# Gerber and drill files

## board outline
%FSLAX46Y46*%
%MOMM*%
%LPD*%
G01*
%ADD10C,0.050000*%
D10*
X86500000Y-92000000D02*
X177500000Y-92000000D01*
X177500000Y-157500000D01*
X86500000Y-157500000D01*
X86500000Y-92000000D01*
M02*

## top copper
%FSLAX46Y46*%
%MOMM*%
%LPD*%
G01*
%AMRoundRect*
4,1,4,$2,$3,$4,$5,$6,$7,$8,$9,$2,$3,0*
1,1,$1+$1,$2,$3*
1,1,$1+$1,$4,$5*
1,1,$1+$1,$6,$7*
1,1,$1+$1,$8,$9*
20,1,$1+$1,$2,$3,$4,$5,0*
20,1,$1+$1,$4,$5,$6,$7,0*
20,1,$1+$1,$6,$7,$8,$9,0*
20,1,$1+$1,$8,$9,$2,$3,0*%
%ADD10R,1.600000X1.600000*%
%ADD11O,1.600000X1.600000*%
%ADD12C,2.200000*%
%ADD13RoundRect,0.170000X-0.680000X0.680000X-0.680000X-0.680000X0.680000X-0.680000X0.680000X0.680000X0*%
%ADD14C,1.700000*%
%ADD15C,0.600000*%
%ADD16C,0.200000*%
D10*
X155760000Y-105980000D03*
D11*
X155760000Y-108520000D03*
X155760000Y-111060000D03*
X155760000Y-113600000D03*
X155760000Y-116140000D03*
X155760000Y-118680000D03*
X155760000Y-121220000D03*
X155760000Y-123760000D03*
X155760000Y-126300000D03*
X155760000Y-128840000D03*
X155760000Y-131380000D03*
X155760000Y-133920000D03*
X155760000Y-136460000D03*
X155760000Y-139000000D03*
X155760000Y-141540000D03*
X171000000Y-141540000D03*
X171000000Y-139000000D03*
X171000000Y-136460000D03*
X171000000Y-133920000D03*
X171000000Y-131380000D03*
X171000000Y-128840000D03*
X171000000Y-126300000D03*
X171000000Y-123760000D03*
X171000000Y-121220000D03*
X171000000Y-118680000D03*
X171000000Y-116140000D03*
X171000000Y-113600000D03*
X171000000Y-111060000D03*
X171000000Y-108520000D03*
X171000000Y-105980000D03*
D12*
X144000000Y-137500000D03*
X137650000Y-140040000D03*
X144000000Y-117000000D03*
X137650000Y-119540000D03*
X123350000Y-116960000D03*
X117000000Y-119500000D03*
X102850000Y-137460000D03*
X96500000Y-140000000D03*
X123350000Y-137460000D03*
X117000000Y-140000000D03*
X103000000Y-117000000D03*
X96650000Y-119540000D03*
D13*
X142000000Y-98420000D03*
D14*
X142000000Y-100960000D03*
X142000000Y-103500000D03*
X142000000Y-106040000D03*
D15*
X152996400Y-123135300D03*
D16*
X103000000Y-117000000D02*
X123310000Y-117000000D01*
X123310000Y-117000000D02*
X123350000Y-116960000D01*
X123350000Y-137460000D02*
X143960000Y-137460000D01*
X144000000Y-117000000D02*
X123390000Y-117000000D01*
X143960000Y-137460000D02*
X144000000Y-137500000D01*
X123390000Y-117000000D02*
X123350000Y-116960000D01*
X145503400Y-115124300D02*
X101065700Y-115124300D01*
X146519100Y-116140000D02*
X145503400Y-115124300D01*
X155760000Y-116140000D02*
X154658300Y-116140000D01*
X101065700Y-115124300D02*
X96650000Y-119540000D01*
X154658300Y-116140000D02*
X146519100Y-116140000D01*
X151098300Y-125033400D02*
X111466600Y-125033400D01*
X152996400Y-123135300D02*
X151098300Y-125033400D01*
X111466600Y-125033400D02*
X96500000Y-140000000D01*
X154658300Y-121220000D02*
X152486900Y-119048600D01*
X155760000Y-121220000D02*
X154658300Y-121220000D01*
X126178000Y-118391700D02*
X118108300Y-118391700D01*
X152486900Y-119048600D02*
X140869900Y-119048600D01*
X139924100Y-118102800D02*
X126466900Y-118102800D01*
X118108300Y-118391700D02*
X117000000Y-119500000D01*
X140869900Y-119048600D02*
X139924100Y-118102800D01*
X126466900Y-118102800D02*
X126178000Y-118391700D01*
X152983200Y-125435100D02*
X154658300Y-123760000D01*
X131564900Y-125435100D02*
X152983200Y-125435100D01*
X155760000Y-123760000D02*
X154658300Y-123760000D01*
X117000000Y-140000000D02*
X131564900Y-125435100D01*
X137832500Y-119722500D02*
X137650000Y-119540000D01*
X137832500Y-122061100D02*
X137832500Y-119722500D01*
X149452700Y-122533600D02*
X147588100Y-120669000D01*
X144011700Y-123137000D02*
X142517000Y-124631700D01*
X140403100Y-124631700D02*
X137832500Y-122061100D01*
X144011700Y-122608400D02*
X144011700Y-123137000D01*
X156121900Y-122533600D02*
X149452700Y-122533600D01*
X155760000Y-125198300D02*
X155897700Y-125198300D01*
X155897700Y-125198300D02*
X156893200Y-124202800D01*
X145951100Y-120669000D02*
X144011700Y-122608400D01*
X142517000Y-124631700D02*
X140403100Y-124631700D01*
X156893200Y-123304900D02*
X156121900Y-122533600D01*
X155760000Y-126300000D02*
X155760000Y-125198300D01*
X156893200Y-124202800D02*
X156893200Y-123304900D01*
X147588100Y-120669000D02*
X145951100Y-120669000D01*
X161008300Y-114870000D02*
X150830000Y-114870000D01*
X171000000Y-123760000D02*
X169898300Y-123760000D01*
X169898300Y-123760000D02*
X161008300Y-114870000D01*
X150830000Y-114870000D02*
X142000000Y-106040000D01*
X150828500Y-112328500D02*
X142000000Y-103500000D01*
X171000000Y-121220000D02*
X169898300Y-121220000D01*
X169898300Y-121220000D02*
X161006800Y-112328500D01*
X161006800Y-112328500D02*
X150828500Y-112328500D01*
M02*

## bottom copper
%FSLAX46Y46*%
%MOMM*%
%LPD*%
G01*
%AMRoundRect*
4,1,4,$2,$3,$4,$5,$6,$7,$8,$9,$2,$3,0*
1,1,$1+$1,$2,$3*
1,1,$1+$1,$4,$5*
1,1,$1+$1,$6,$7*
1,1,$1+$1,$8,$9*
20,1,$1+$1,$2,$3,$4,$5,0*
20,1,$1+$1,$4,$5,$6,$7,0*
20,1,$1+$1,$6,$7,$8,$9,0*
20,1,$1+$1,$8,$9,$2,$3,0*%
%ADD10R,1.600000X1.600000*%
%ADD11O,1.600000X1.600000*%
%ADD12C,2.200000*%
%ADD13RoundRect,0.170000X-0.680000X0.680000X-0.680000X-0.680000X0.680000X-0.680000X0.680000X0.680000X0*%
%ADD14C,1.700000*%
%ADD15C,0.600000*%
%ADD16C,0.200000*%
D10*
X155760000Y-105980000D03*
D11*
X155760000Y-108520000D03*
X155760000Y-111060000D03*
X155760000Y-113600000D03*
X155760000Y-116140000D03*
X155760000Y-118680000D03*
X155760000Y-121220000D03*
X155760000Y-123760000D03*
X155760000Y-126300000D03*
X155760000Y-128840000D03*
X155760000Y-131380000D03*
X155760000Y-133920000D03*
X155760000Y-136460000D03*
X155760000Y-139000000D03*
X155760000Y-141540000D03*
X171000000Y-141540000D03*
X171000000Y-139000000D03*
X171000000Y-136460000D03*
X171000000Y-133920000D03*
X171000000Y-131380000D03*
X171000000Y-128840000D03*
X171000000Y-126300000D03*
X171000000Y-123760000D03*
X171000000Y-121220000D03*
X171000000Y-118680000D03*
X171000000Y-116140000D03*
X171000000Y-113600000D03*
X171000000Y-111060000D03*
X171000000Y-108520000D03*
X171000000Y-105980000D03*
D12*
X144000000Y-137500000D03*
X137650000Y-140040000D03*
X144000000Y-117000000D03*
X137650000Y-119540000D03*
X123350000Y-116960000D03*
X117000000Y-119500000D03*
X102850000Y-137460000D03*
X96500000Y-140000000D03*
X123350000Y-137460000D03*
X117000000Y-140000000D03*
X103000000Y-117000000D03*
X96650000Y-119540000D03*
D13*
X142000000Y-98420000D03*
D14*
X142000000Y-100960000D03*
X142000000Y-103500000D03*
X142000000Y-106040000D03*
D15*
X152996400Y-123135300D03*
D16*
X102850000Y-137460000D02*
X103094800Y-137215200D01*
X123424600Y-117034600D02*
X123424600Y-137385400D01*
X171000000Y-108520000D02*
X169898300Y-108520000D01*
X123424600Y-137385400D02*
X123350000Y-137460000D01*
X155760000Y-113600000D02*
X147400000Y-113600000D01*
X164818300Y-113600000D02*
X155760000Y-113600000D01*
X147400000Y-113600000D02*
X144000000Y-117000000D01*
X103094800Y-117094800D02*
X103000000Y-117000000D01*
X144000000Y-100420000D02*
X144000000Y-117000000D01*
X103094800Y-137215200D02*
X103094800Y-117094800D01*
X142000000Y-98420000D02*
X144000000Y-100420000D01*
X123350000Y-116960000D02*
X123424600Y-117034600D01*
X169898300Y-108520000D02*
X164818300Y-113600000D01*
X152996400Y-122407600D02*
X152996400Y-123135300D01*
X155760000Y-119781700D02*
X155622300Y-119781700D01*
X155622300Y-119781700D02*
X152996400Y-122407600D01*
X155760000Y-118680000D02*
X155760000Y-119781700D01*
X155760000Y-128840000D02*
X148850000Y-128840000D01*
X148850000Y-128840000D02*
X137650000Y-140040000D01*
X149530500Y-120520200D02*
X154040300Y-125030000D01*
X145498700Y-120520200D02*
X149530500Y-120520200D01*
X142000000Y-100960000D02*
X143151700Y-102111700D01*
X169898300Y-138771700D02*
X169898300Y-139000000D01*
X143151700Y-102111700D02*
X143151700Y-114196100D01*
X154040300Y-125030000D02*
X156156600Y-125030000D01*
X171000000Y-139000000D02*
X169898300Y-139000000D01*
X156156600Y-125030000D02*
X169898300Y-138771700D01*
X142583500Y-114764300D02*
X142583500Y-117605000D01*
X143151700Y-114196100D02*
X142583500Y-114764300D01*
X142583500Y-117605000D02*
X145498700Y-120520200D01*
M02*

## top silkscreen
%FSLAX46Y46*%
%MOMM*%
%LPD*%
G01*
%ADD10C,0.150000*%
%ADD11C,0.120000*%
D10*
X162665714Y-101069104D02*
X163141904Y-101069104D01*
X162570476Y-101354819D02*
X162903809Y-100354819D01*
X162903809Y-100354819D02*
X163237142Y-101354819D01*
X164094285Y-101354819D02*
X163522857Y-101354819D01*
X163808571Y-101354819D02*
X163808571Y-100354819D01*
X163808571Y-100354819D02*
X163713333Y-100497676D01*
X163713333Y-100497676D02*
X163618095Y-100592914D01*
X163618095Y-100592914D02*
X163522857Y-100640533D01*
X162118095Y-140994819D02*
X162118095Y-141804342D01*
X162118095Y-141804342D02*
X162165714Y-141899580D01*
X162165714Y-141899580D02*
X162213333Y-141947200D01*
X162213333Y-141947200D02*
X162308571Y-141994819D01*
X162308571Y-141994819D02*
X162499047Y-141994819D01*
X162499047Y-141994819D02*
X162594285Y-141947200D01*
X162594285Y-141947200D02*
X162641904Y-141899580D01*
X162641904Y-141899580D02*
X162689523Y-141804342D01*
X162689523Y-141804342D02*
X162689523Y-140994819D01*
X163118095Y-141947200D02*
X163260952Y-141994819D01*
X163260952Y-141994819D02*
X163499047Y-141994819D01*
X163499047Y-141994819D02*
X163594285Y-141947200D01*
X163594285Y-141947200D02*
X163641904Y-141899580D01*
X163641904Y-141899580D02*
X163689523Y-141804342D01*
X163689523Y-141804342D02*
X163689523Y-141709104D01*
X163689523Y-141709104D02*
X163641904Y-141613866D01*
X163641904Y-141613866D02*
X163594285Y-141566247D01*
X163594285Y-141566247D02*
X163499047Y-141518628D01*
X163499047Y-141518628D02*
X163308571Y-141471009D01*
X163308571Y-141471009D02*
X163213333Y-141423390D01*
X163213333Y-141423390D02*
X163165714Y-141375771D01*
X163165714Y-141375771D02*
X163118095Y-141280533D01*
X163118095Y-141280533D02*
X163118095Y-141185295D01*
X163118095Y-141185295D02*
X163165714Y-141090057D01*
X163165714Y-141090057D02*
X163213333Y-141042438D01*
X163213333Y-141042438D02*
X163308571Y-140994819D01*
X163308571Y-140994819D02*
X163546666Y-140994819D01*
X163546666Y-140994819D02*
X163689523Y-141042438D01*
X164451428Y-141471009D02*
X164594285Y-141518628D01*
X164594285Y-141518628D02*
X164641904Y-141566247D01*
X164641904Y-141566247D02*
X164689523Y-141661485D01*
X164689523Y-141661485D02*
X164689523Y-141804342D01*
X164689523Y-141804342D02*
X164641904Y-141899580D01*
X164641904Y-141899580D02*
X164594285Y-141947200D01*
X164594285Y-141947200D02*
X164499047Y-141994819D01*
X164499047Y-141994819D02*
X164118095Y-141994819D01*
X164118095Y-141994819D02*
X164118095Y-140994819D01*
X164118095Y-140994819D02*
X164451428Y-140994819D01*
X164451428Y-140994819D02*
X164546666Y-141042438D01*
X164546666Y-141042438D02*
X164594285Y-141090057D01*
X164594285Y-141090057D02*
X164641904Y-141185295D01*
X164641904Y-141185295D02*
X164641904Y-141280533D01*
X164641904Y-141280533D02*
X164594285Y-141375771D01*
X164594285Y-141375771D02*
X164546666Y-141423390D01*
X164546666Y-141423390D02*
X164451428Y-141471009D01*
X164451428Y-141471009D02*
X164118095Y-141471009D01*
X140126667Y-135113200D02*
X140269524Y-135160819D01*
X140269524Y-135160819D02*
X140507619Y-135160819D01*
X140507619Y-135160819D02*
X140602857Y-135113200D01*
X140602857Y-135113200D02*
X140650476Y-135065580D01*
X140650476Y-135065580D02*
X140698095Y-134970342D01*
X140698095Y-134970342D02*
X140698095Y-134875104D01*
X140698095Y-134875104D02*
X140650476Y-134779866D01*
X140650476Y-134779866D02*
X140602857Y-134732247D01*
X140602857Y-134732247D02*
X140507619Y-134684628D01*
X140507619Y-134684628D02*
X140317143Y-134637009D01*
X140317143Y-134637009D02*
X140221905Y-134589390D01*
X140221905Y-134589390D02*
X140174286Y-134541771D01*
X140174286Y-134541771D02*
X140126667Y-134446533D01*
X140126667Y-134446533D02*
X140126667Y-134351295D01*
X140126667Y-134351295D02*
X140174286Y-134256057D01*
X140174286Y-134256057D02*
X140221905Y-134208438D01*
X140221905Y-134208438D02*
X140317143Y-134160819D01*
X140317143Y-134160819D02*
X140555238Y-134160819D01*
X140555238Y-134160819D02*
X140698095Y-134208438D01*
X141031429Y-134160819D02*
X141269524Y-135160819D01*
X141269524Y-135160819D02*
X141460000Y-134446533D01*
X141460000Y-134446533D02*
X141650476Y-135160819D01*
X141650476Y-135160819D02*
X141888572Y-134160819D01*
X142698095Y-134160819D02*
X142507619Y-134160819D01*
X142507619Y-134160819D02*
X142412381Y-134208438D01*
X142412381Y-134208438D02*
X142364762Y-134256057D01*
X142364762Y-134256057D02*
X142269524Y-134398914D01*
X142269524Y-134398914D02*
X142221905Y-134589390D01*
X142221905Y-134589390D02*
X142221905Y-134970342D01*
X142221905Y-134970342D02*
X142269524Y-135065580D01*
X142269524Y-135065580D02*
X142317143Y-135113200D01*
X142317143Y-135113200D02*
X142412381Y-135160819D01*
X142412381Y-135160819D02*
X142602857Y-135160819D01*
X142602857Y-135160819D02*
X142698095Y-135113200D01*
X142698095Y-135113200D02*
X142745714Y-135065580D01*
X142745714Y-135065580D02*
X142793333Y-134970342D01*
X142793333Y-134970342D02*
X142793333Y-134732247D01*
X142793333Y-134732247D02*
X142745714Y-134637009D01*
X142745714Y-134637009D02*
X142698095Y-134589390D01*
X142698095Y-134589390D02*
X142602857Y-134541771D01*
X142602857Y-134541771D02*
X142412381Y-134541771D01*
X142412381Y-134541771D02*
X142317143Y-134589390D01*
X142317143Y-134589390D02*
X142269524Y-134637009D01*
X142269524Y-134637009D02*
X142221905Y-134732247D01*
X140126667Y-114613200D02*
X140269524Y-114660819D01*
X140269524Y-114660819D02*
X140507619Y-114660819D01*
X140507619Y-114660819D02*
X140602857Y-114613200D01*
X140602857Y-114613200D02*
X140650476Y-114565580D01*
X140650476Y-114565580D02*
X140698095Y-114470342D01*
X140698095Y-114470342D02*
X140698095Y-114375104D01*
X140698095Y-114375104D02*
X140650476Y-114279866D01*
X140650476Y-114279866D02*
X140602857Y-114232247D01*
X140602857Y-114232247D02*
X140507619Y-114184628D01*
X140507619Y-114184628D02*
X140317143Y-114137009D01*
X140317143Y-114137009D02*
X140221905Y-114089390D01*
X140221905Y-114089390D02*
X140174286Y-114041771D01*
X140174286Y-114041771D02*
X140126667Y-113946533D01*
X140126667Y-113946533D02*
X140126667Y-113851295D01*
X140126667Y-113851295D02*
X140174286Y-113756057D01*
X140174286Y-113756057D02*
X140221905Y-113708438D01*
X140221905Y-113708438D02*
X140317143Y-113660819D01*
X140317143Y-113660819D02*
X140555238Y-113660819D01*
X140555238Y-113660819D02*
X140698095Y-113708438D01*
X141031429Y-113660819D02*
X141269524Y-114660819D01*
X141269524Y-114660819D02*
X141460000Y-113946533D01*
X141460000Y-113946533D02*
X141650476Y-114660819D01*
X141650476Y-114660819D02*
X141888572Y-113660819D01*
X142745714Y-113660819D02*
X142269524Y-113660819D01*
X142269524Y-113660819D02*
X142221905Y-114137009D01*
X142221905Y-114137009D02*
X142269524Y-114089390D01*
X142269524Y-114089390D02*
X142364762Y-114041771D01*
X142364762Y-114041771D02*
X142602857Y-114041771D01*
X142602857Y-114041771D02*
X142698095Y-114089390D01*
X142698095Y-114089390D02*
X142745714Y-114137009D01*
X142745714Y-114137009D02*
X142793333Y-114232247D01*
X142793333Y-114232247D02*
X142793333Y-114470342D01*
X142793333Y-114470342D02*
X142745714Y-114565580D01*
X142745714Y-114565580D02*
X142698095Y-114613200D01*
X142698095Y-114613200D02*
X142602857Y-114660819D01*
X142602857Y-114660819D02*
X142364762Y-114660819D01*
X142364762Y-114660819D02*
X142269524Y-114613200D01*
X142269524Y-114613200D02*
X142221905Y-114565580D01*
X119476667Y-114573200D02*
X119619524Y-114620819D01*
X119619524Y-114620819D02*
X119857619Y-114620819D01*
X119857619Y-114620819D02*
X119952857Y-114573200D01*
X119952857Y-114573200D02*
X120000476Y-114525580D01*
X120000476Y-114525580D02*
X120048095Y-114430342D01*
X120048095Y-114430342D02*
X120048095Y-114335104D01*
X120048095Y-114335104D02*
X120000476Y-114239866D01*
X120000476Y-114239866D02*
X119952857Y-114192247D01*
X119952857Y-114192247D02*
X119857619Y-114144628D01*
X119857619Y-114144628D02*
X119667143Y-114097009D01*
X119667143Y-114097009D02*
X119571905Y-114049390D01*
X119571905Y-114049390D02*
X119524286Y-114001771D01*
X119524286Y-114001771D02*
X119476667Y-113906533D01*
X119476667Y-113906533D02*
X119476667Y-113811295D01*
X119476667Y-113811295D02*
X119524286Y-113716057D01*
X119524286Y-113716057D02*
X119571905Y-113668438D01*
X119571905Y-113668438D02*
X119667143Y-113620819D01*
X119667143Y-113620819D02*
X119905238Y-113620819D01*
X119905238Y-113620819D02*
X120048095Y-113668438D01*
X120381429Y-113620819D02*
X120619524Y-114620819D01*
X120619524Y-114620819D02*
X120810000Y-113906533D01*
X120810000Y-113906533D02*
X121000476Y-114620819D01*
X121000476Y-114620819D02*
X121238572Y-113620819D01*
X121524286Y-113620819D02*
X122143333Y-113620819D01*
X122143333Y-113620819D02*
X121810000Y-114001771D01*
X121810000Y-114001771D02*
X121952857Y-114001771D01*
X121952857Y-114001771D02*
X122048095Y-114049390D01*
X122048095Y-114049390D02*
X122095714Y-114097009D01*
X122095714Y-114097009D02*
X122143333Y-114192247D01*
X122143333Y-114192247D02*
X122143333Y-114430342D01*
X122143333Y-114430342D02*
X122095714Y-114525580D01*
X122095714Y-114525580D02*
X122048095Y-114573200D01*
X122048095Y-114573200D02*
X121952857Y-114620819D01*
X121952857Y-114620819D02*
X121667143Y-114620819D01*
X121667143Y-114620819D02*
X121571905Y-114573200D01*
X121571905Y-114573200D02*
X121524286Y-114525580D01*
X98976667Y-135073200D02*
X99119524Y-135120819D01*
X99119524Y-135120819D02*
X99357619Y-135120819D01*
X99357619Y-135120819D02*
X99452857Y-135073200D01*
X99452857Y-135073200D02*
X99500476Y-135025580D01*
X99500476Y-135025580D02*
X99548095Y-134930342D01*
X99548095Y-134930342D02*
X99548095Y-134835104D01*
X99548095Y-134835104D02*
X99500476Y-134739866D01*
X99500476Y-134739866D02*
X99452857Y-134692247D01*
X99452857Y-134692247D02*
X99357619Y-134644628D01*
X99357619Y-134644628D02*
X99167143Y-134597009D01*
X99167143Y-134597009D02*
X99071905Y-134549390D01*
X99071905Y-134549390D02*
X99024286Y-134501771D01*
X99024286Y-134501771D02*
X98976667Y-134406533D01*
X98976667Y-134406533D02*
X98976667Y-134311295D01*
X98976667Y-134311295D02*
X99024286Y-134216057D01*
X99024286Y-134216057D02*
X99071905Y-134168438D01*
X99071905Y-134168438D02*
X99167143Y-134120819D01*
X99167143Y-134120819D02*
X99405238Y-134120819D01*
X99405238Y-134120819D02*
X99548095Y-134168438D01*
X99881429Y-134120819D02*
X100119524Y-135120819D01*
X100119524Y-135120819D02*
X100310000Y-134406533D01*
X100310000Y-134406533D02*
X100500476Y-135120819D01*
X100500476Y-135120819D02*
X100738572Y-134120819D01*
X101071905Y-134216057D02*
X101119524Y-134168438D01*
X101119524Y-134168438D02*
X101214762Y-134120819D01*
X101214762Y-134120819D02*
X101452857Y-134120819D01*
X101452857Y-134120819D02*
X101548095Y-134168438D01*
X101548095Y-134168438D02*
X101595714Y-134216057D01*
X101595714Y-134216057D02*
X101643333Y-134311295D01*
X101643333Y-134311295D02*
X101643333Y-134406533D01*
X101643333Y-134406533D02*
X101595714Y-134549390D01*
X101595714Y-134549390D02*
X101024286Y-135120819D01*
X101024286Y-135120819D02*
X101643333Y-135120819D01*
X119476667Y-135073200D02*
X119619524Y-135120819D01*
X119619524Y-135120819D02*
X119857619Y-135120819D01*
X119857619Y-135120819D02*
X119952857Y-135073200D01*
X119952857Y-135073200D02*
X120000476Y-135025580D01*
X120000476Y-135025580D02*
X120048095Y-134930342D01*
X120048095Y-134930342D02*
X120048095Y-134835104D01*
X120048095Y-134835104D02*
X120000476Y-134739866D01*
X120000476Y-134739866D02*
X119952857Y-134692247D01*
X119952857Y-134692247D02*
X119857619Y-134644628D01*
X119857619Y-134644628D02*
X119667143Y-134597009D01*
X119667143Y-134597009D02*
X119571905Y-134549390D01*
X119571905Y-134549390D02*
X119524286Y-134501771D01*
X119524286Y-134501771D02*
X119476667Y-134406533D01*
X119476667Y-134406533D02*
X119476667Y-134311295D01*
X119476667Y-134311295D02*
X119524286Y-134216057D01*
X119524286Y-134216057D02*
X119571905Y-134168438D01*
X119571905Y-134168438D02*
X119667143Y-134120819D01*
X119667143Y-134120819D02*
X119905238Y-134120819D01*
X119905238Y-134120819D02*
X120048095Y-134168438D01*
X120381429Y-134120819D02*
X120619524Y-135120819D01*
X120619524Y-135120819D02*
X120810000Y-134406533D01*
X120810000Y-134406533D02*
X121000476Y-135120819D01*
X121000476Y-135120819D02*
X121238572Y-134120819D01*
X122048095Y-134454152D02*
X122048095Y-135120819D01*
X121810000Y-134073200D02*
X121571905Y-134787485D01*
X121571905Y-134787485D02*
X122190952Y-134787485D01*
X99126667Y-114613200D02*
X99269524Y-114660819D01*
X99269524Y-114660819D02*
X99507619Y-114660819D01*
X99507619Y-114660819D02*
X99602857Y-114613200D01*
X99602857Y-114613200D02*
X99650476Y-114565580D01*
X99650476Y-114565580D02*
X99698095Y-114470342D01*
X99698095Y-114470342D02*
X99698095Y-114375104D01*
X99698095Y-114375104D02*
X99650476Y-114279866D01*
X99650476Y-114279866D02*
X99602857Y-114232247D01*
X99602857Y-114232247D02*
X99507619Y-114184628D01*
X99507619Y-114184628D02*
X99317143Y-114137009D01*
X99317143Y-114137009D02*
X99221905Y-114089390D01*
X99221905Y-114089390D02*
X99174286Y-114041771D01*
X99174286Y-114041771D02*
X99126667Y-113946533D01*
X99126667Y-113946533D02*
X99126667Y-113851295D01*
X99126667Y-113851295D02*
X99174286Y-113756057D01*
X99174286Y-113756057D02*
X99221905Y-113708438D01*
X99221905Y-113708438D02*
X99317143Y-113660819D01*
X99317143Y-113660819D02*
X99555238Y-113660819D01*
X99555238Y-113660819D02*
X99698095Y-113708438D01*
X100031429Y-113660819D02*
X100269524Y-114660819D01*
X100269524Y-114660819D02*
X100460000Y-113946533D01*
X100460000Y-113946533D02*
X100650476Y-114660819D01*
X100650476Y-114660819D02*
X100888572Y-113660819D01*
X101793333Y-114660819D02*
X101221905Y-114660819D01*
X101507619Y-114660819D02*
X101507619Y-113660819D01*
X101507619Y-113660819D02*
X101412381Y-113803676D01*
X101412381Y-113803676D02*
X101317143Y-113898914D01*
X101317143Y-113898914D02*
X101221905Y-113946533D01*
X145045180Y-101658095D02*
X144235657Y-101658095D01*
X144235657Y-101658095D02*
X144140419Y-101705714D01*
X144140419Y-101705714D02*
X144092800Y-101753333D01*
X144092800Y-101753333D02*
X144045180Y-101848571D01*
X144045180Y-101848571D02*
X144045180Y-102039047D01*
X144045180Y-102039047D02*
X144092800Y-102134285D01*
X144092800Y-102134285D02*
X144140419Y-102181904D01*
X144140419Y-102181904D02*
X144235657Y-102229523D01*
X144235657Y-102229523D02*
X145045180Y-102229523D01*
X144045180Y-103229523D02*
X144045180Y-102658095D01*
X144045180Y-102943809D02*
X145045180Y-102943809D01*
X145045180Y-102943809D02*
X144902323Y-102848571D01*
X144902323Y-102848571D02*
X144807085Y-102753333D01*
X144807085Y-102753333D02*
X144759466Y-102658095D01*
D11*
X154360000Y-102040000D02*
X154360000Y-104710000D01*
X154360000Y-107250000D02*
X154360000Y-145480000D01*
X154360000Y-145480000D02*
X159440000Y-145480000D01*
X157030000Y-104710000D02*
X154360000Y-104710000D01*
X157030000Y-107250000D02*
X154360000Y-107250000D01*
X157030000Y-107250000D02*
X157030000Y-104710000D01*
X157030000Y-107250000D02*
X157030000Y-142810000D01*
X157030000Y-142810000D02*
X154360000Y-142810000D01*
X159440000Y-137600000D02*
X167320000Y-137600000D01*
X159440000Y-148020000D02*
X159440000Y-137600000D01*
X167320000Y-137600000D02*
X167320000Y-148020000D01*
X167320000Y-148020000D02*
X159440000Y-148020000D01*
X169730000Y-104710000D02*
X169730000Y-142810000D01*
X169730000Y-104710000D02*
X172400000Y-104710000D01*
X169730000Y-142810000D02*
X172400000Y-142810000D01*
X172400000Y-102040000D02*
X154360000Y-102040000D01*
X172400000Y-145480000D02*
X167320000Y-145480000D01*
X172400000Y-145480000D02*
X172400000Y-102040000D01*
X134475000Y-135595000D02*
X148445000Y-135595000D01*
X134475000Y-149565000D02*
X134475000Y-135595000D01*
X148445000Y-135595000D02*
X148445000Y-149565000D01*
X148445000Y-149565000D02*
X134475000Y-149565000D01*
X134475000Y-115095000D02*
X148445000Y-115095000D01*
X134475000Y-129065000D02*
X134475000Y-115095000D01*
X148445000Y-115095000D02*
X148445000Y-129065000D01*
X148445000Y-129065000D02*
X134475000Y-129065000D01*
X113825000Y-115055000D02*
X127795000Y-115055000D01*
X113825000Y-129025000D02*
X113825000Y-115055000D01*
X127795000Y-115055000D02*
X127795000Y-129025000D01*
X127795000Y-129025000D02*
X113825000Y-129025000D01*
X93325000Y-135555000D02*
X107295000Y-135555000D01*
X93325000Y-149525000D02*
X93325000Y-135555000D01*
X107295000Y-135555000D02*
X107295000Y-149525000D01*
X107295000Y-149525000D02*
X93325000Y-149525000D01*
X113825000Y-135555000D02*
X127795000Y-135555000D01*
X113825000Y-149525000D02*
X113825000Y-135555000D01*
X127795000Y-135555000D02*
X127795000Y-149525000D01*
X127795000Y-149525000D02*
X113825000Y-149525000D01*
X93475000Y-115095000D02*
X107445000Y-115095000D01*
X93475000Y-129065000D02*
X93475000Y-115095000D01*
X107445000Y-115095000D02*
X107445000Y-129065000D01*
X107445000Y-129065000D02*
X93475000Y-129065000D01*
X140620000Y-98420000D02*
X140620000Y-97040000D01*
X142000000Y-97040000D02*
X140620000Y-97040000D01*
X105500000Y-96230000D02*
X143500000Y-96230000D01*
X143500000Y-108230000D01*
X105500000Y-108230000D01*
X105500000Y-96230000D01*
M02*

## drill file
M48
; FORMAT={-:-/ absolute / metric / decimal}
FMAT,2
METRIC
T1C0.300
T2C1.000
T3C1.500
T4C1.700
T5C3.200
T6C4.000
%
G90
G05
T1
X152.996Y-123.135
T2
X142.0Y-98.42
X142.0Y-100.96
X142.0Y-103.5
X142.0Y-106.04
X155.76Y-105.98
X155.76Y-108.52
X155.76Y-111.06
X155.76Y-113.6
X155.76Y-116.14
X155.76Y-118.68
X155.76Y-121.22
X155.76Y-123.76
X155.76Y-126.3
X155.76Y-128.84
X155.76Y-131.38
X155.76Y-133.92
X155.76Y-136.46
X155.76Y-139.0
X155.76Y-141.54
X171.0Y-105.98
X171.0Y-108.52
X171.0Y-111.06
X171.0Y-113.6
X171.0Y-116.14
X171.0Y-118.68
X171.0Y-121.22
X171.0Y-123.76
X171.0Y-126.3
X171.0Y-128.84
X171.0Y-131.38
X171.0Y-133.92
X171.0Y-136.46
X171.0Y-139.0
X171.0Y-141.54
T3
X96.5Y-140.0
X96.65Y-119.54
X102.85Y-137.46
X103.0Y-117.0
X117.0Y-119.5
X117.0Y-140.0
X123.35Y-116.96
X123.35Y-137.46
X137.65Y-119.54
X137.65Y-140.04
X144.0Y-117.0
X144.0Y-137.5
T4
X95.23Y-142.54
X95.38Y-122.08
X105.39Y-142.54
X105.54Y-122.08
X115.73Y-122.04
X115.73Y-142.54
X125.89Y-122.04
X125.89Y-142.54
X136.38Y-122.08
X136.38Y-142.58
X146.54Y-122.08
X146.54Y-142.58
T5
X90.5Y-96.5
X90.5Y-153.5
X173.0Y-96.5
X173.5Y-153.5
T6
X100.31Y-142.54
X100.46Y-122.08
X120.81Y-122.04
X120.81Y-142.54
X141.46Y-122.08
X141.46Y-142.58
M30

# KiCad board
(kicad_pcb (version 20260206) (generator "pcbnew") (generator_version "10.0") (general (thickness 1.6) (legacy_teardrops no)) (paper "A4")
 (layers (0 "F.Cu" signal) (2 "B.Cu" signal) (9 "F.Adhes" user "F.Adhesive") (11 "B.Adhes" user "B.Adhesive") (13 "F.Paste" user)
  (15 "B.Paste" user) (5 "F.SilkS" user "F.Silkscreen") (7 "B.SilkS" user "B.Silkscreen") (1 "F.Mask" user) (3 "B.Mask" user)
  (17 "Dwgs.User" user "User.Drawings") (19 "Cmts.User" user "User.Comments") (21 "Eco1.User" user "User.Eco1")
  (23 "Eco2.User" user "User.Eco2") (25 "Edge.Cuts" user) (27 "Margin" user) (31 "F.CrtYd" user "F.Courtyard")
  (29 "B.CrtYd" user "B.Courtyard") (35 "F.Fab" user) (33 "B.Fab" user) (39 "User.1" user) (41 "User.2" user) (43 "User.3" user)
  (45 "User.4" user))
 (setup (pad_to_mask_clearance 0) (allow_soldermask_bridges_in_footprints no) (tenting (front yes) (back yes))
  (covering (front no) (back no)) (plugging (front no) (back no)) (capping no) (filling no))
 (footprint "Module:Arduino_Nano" (layer "F.Cu") (at 155.76 105.98)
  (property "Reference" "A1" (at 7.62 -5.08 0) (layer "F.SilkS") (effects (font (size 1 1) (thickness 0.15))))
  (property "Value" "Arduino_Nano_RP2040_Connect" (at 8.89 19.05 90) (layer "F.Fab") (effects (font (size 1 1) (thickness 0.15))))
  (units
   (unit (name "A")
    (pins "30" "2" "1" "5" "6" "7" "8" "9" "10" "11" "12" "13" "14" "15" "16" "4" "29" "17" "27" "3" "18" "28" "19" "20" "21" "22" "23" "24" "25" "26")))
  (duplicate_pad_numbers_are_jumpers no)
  (fp_line (start -1.4 -3.94) (end -1.4 -1.27) (stroke (width 0.12) (type solid)) (layer "F.SilkS"))
  (fp_line (start -1.4 1.27) (end -1.4 39.5) (stroke (width 0.12) (type solid)) (layer "F.SilkS"))
  (fp_line (start -1.4 39.5) (end 3.68 39.5) (stroke (width 0.12) (type solid)) (layer "F.SilkS"))
  (fp_line (start 1.27 -1.27) (end -1.4 -1.27) (stroke (width 0.12) (type solid)) (layer "F.SilkS"))
  (fp_line (start 1.27 1.27) (end -1.4 1.27) (stroke (width 0.12) (type solid)) (layer "F.SilkS"))
  (fp_line (start 1.27 1.27) (end 1.27 -1.27) (stroke (width 0.12) (type solid)) (layer "F.SilkS"))
  (fp_line (start 1.27 1.27) (end 1.27 36.83) (stroke (width 0.12) (type solid)) (layer "F.SilkS"))
  (fp_line (start 1.27 36.83) (end -1.4 36.83) (stroke (width 0.12) (type solid)) (layer "F.SilkS"))
  (fp_line (start 3.68 31.62) (end 11.56 31.62) (stroke (width 0.12) (type solid)) (layer "F.SilkS"))
  (fp_line (start 3.68 42.04) (end 3.68 31.62) (stroke (width 0.12) (type solid)) (layer "F.SilkS"))
  (fp_line (start 11.56 31.62) (end 11.56 42.04) (stroke (width 0.12) (type solid)) (layer "F.SilkS"))
  (fp_line (start 11.56 42.04) (end 3.68 42.04) (stroke (width 0.12) (type solid)) (layer "F.SilkS"))
  (fp_line (start 13.97 -1.27) (end 13.97 36.83) (stroke (width 0.12) (type solid)) (layer "F.SilkS"))
  (fp_line (start 13.97 -1.27) (end 16.64 -1.27) (stroke (width 0.12) (type solid)) (layer "F.SilkS"))
  (fp_line (start 13.97 36.83) (end 16.64 36.83) (stroke (width 0.12) (type solid)) (layer "F.SilkS"))
  (fp_line (start 16.64 -3.94) (end -1.4 -3.94) (stroke (width 0.12) (type solid)) (layer "F.SilkS"))
  (fp_line (start 16.64 39.5) (end 11.56 39.5) (stroke (width 0.12) (type solid)) (layer "F.SilkS"))
  (fp_line (start 16.64 39.5) (end 16.64 -3.94) (stroke (width 0.12) (type solid)) (layer "F.SilkS"))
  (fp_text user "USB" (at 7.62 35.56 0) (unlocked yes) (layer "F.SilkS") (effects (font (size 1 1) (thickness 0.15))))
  (pad "1" thru_hole rect (at 0 0) (size 1.6 1.6) (drill 1) (layers "*.Cu" "*.Mask") (remove_unused_layers no)
   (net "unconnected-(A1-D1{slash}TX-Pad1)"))
  (pad "2" thru_hole oval (at 0 2.54) (size 1.6 1.6) (drill 1) (layers "*.Cu" "*.Mask") (remove_unused_layers no)
   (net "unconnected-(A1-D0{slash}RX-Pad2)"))
  (pad "3" thru_hole oval (at 0 5.08) (size 1.6 1.6) (drill 1) (layers "*.Cu" "*.Mask") (remove_unused_layers no)
   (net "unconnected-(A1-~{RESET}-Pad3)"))
  (pad "4" thru_hole oval (at 0 7.62) (size 1.6 1.6) (drill 1) (layers "*.Cu" "*.Mask") (remove_unused_layers no) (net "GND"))
  (pad "5" thru_hole oval (at 0 10.16) (size 1.6 1.6) (drill 1) (layers "*.Cu" "*.Mask") (remove_unused_layers no) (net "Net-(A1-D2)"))
  (pad "6" thru_hole oval (at 0 12.7) (size 1.6 1.6) (drill 1) (layers "*.Cu" "*.Mask") (remove_unused_layers no) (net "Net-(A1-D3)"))
  (pad "7" thru_hole oval (at 0 15.24) (size 1.6 1.6) (drill 1) (layers "*.Cu" "*.Mask") (remove_unused_layers no) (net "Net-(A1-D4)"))
  (pad "8" thru_hole oval (at 0 17.78) (size 1.6 1.6) (drill 1) (layers "*.Cu" "*.Mask") (remove_unused_layers no) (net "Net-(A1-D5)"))
  (pad "9" thru_hole oval (at 0 20.32) (size 1.6 1.6) (drill 1) (layers "*.Cu" "*.Mask") (remove_unused_layers no) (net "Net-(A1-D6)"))
  (pad "10" thru_hole oval (at 0 22.86) (size 1.6 1.6) (drill 1) (layers "*.Cu" "*.Mask") (remove_unused_layers no) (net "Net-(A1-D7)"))
  (pad "11" thru_hole oval (at 0 25.4) (size 1.6 1.6) (drill 1) (layers "*.Cu" "*.Mask") (remove_unused_layers no)
   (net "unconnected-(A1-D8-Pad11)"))
  (pad "12" thru_hole oval (at 0 27.94) (size 1.6 1.6) (drill 1) (layers "*.Cu" "*.Mask") (remove_unused_layers no)
   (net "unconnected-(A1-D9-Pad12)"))
  (pad "13" thru_hole oval (at 0 30.48) (size 1.6 1.6) (drill 1) (layers "*.Cu" "*.Mask") (remove_unused_layers no)
   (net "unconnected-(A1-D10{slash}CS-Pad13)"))
  (pad "14" thru_hole oval (at 0 33.02) (size 1.6 1.6) (drill 1) (layers "*.Cu" "*.Mask") (remove_unused_layers no)
   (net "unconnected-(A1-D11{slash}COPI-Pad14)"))
  (pad "15" thru_hole oval (at 0 35.56) (size 1.6 1.6) (drill 1) (layers "*.Cu" "*.Mask") (remove_unused_layers no)
   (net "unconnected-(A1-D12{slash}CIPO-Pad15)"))
  (pad "16" thru_hole oval (at 15.24 35.56) (size 1.6 1.6) (drill 1) (layers "*.Cu" "*.Mask") (remove_unused_layers no)
   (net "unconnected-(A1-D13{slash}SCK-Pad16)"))
  (pad "17" thru_hole oval (at 15.24 33.02) (size 1.6 1.6) (drill 1) (layers "*.Cu" "*.Mask") (remove_unused_layers no) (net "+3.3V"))
  (pad "18" thru_hole oval (at 15.24 30.48) (size 1.6 1.6) (drill 1) (layers "*.Cu" "*.Mask") (remove_unused_layers no)
   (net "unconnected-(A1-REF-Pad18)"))
  (pad "19" thru_hole oval (at 15.24 27.94) (size 1.6 1.6) (drill 1) (layers "*.Cu" "*.Mask") (remove_unused_layers no)
   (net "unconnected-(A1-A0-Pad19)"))
  (pad "20" thru_hole oval (at 15.24 25.4) (size 1.6 1.6) (drill 1) (layers "*.Cu" "*.Mask") (remove_unused_layers no)
   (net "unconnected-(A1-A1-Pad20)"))
  (pad "21" thru_hole oval (at 15.24 22.86) (size 1.6 1.6) (drill 1) (layers "*.Cu" "*.Mask") (remove_unused_layers no)
   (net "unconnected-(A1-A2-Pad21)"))
  (pad "22" thru_hole oval (at 15.24 20.32) (size 1.6 1.6) (drill 1) (layers "*.Cu" "*.Mask") (remove_unused_layers no)
   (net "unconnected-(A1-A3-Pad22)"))
  (pad "23" thru_hole oval (at 15.24 17.78) (size 1.6 1.6) (drill 1) (layers "*.Cu" "*.Mask") (remove_unused_layers no)
   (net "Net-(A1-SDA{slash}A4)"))
  (pad "24" thru_hole oval (at 15.24 15.24) (size 1.6 1.6) (drill 1) (layers "*.Cu" "*.Mask") (remove_unused_layers no)
   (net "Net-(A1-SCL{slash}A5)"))
  (pad "25" thru_hole oval (at 15.24 12.7) (size 1.6 1.6) (drill 1) (layers "*.Cu" "*.Mask") (remove_unused_layers no)
   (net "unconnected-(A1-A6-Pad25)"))
  (pad "26" thru_hole oval (at 15.24 10.16) (size 1.6 1.6) (drill 1) (layers "*.Cu" "*.Mask") (remove_unused_layers no)
   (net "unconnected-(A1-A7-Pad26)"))
  (pad "27" thru_hole oval (at 15.24 7.62) (size 1.6 1.6) (drill 1) (layers "*.Cu" "*.Mask") (remove_unused_layers no)
   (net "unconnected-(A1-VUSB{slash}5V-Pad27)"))
  (pad "28" thru_hole oval (at 15.24 5.08) (size 1.6 1.6) (drill 1) (layers "*.Cu" "*.Mask") (remove_unused_layers no)
   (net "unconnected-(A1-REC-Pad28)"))
  (pad "29" thru_hole oval (at 15.24 2.54) (size 1.6 1.6) (drill 1) (layers "*.Cu" "*.Mask") (remove_unused_layers no) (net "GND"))
  (pad "30" thru_hole oval (at 15.24 0) (size 1.6 1.6) (drill 1) (layers "*.Cu" "*.Mask") (remove_unused_layers no)
   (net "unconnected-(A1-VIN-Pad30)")))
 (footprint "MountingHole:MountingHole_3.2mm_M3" (layer "F.Cu") (at 173.5 153.5)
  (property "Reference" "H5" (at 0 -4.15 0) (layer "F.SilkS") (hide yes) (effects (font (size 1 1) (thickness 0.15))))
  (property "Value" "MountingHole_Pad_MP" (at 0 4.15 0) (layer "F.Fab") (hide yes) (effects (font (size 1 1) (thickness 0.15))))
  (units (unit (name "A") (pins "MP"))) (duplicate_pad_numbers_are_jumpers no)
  (pad "" np_thru_hole circle (at 0 0) (size 3.2 3.2) (drill 3.2) (layers "*.Cu" "*.Mask")))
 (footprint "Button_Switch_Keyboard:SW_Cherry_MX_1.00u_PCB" (layer "F.Cu") (at 144 137.5)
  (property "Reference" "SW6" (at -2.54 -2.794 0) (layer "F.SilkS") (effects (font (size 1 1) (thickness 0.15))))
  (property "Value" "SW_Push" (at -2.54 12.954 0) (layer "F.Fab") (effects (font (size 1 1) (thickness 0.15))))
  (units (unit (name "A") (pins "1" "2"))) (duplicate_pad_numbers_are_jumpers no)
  (fp_line (start -9.525 -1.905) (end 4.445 -1.905) (stroke (width 0.12) (type solid)) (layer "F.SilkS"))
  (fp_line (start -9.525 12.065) (end -9.525 -1.905) (stroke (width 0.12) (type solid)) (layer "F.SilkS"))
  (fp_line (start 4.445 -1.905) (end 4.445 12.065) (stroke (width 0.12) (type solid)) (layer "F.SilkS"))
  (fp_line (start 4.445 12.065) (end -9.525 12.065) (stroke (width 0.12) (type solid)) (layer "F.SilkS"))
  (pad "" np_thru_hole circle (at -7.62 5.08) (size 1.7 1.7) (drill 1.7) (layers "*.Cu" "*.Mask"))
  (pad "" np_thru_hole circle (at -2.54 5.08) (size 4 4) (drill 4) (layers "*.Cu" "*.Mask"))
  (pad "" np_thru_hole circle (at 2.54 5.08) (size 1.7 1.7) (drill 1.7) (layers "*.Cu" "*.Mask"))
  (pad "1" thru_hole circle (at 0 0) (size 2.2 2.2) (drill 1.5) (layers "*.Cu" "*.Mask") (remove_unused_layers no) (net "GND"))
  (pad "2" thru_hole circle (at -6.35 2.54) (size 2.2 2.2) (drill 1.5) (layers "*.Cu" "*.Mask") (remove_unused_layers no)
   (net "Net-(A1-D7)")))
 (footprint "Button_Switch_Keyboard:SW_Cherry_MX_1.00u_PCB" (layer "F.Cu") (at 144 117)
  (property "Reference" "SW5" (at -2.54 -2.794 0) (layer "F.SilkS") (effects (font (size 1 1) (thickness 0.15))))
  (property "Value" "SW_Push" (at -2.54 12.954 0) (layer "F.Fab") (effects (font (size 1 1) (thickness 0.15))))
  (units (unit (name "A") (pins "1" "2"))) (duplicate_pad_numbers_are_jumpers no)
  (fp_line (start -9.525 -1.905) (end 4.445 -1.905) (stroke (width 0.12) (type solid)) (layer "F.SilkS"))
  (fp_line (start -9.525 12.065) (end -9.525 -1.905) (stroke (width 0.12) (type solid)) (layer "F.SilkS"))
  (fp_line (start 4.445 -1.905) (end 4.445 12.065) (stroke (width 0.12) (type solid)) (layer "F.SilkS"))
  (fp_line (start 4.445 12.065) (end -9.525 12.065) (stroke (width 0.12) (type solid)) (layer "F.SilkS"))
  (pad "" np_thru_hole circle (at -7.62 5.08) (size 1.7 1.7) (drill 1.7) (layers "*.Cu" "*.Mask"))
  (pad "" np_thru_hole circle (at -2.54 5.08) (size 4 4) (drill 4) (layers "*.Cu" "*.Mask"))
  (pad "" np_thru_hole circle (at 2.54 5.08) (size 1.7 1.7) (drill 1.7) (layers "*.Cu" "*.Mask"))
  (pad "1" thru_hole circle (at 0 0) (size 2.2 2.2) (drill 1.5) (layers "*.Cu" "*.Mask") (remove_unused_layers no) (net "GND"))
  (pad "2" thru_hole circle (at -6.35 2.54) (size 2.2 2.2) (drill 1.5) (layers "*.Cu" "*.Mask") (remove_unused_layers no)
   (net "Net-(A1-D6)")))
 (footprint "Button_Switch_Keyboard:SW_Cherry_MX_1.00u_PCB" (layer "F.Cu") (at 123.35 116.96)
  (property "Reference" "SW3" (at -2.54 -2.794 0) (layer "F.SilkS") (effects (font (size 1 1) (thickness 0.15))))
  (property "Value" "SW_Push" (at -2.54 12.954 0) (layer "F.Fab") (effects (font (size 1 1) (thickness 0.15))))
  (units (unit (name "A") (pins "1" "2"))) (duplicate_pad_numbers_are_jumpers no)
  (fp_line (start -9.525 -1.905) (end 4.445 -1.905) (stroke (width 0.12) (type solid)) (layer "F.SilkS"))
  (fp_line (start -9.525 12.065) (end -9.525 -1.905) (stroke (width 0.12) (type solid)) (layer "F.SilkS"))
  (fp_line (start 4.445 -1.905) (end 4.445 12.065) (stroke (width 0.12) (type solid)) (layer "F.SilkS"))
  (fp_line (start 4.445 12.065) (end -9.525 12.065) (stroke (width 0.12) (type solid)) (layer "F.SilkS"))
  (pad "" np_thru_hole circle (at -7.62 5.08) (size 1.7 1.7) (drill 1.7) (layers "*.Cu" "*.Mask"))
  (pad "" np_thru_hole circle (at -2.54 5.08) (size 4 4) (drill 4) (layers "*.Cu" "*.Mask"))
  (pad "" np_thru_hole circle (at 2.54 5.08) (size 1.7 1.7) (drill 1.7) (layers "*.Cu" "*.Mask"))
  (pad "1" thru_hole circle (at 0 0) (size 2.2 2.2) (drill 1.5) (layers "*.Cu" "*.Mask") (remove_unused_layers no) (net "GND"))
  (pad "2" thru_hole circle (at -6.35 2.54) (size 2.2 2.2) (drill 1.5) (layers "*.Cu" "*.Mask") (remove_unused_layers no)
   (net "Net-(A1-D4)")))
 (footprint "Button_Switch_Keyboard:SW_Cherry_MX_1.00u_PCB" (layer "F.Cu") (at 102.85 137.46)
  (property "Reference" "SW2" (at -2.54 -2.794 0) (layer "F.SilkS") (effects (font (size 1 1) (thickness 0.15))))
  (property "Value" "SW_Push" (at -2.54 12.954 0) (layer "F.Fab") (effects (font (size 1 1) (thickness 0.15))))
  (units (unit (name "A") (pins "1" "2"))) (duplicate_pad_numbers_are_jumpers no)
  (fp_line (start -9.525 -1.905) (end 4.445 -1.905) (stroke (width 0.12) (type solid)) (layer "F.SilkS"))
  (fp_line (start -9.525 12.065) (end -9.525 -1.905) (stroke (width 0.12) (type solid)) (layer "F.SilkS"))
  (fp_line (start 4.445 -1.905) (end 4.445 12.065) (stroke (width 0.12) (type solid)) (layer "F.SilkS"))
  (fp_line (start 4.445 12.065) (end -9.525 12.065) (stroke (width 0.12) (type solid)) (layer "F.SilkS"))
  (pad "" np_thru_hole circle (at -7.62 5.08) (size 1.7 1.7) (drill 1.7) (layers "*.Cu" "*.Mask"))
  (pad "" np_thru_hole circle (at -2.54 5.08) (size 4 4) (drill 4) (layers "*.Cu" "*.Mask"))
  (pad "" np_thru_hole circle (at 2.54 5.08) (size 1.7 1.7) (drill 1.7) (layers "*.Cu" "*.Mask"))
  (pad "1" thru_hole circle (at 0 0) (size 2.2 2.2) (drill 1.5) (layers "*.Cu" "*.Mask") (remove_unused_layers no) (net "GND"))
  (pad "2" thru_hole circle (at -6.35 2.54) (size 2.2 2.2) (drill 1.5) (layers "*.Cu" "*.Mask") (remove_unused_layers no)
   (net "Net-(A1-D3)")))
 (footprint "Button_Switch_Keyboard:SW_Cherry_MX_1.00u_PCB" (layer "F.Cu") (at 123.35 137.46)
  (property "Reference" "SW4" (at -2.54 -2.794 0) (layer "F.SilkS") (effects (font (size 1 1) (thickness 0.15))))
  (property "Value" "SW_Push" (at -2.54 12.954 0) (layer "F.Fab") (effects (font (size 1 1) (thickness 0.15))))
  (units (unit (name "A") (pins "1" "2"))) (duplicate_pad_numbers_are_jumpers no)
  (fp_line (start -9.525 -1.905) (end 4.445 -1.905) (stroke (width 0.12) (type solid)) (layer "F.SilkS"))
  (fp_line (start -9.525 12.065) (end -9.525 -1.905) (stroke (width 0.12) (type solid)) (layer "F.SilkS"))
  (fp_line (start 4.445 -1.905) (end 4.445 12.065) (stroke (width 0.12) (type solid)) (layer "F.SilkS"))
  (fp_line (start 4.445 12.065) (end -9.525 12.065) (stroke (width 0.12) (type solid)) (layer "F.SilkS"))
  (pad "" np_thru_hole circle (at -7.62 5.08) (size 1.7 1.7) (drill 1.7) (layers "*.Cu" "*.Mask"))
  (pad "" np_thru_hole circle (at -2.54 5.08) (size 4 4) (drill 4) (layers "*.Cu" "*.Mask"))
  (pad "" np_thru_hole circle (at 2.54 5.08) (size 1.7 1.7) (drill 1.7) (layers "*.Cu" "*.Mask"))
  (pad "1" thru_hole circle (at 0 0) (size 2.2 2.2) (drill 1.5) (layers "*.Cu" "*.Mask") (remove_unused_layers no) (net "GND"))
  (pad "2" thru_hole circle (at -6.35 2.54) (size 2.2 2.2) (drill 1.5) (layers "*.Cu" "*.Mask") (remove_unused_layers no)
   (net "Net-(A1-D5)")))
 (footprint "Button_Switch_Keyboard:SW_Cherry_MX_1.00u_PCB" (layer "F.Cu") (at 103 117)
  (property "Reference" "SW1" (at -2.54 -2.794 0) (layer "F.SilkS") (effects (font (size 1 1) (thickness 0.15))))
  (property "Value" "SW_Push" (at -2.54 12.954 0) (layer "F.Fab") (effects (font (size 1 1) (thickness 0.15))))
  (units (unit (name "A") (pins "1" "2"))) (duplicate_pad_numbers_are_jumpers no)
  (fp_line (start -9.525 -1.905) (end 4.445 -1.905) (stroke (width 0.12) (type solid)) (layer "F.SilkS"))
  (fp_line (start -9.525 12.065) (end -9.525 -1.905) (stroke (width 0.12) (type solid)) (layer "F.SilkS"))
  (fp_line (start 4.445 -1.905) (end 4.445 12.065) (stroke (width 0.12) (type solid)) (layer "F.SilkS"))
  (fp_line (start 4.445 12.065) (end -9.525 12.065) (stroke (width 0.12) (type solid)) (layer "F.SilkS"))
  (pad "" np_thru_hole circle (at -7.62 5.08) (size 1.7 1.7) (drill 1.7) (layers "*.Cu" "*.Mask"))
  (pad "" np_thru_hole circle (at -2.54 5.08) (size 4 4) (drill 4) (layers "*.Cu" "*.Mask"))
  (pad "" np_thru_hole circle (at 2.54 5.08) (size 1.7 1.7) (drill 1.7) (layers "*.Cu" "*.Mask"))
  (pad "1" thru_hole circle (at 0 0) (size 2.2 2.2) (drill 1.5) (layers "*.Cu" "*.Mask") (remove_unused_layers no) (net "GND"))
  (pad "2" thru_hole circle (at -6.35 2.54) (size 2.2 2.2) (drill 1.5) (layers "*.Cu" "*.Mask") (remove_unused_layers no)
   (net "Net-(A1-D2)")))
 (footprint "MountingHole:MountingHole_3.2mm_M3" (layer "F.Cu") (at 90.5 96.5)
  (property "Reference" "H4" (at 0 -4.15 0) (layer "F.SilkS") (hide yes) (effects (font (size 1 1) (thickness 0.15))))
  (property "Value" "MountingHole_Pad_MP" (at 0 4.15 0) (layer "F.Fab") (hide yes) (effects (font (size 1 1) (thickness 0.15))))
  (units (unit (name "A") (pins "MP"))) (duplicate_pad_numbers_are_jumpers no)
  (pad "" np_thru_hole circle (at 0 0) (size 3.2 3.2) (drill 3.2) (layers "*.Cu" "*.Mask")))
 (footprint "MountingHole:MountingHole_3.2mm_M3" (layer "F.Cu") (at 90.5 153.5)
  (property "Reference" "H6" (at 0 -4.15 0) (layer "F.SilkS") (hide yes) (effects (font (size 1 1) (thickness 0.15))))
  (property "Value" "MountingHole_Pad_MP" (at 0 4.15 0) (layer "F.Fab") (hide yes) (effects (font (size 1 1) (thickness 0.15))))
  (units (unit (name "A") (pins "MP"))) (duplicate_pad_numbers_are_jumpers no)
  (pad "" np_thru_hole circle (at 0 0) (size 3.2 3.2) (drill 3.2) (layers "*.Cu" "*.Mask")))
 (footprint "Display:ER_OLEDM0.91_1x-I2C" (layer "F.Cu") (at 142 98.42 -90)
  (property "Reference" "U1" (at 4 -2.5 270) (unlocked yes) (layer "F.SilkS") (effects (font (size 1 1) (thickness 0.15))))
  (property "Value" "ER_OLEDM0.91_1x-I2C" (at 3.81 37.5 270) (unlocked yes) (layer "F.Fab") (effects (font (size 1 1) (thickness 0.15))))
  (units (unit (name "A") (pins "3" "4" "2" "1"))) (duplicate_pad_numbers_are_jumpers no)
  (fp_line (start 0 1.38) (end -1.38 1.38) (stroke (width 0.12) (type solid)) (layer "F.SilkS"))
  (fp_line (start -1.38 0) (end -1.38 1.38) (stroke (width 0.12) (type solid)) (layer "F.SilkS"))
  (fp_rect (start -2.19 -1.5) (end 9.81 36.5) (stroke (width 0.12) (type solid)) (fill no) (layer "F.SilkS"))
  (pad "1" thru_hole roundrect (at 0 0 270) (size 1.7 1.7) (drill 1) (layers "*.Cu" "*.Mask") (remove_unused_layers no)
   (roundrect_rratio 0.1) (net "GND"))
  (pad "2" thru_hole circle (at 2.54 0 270) (size 1.7 1.7) (drill 1) (layers "*.Cu" "*.Mask") (remove_unused_layers no) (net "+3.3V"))
  (pad "3" thru_hole circle (at 5.08 0 270) (size 1.7 1.7) (drill 1) (layers "*.Cu" "*.Mask") (remove_unused_layers no)
   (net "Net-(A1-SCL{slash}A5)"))
  (pad "4" thru_hole circle (at 7.62 0 270) (size 1.7 1.7) (drill 1) (layers "*.Cu" "*.Mask") (remove_unused_layers no)
   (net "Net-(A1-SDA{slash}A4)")))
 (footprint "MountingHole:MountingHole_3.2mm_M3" (layer "F.Cu") (at 173 96.5)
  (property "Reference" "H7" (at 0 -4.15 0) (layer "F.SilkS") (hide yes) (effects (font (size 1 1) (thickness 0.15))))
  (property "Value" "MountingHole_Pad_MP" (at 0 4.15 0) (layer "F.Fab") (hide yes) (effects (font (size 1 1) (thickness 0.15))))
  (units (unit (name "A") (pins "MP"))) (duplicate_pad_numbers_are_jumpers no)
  (pad "" np_thru_hole circle (at 0 0) (size 3.2 3.2) (drill 3.2) (layers "*.Cu" "*.Mask")))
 (gr_rect (start 86.5 92) (end 177.5 157.5) (stroke (width 0.05) (type default)) (fill no) (layer "Edge.Cuts"))
 (segment (start 103 117) (end 123.31 117) (width 0.2) (layer "F.Cu") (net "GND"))
 (segment (start 123.31 117) (end 123.35 116.96) (width 0.2) (layer "F.Cu") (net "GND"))
 (segment (start 123.35 137.46) (end 143.96 137.46) (width 0.2) (layer "F.Cu") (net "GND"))
 (segment (start 144 117) (end 123.39 117) (width 0.2) (layer "F.Cu") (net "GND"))
 (segment (start 143.96 137.46) (end 144 137.5) (width 0.2) (layer "F.Cu") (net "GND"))
 (segment (start 123.39 117) (end 123.35 116.96) (width 0.2) (layer "F.Cu") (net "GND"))
 (segment (start 102.85 137.46) (end 103.0948 137.2152) (width 0.2) (layer "B.Cu") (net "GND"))
 (segment (start 123.4246 117.0346) (end 123.4246 137.3854) (width 0.2) (layer "B.Cu") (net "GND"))
 (segment (start 171 108.52) (end 169.8983 108.52) (width 0.2) (layer "B.Cu") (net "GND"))
 (segment (start 123.4246 137.3854) (end 123.35 137.46) (width 0.2) (layer "B.Cu") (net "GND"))
 (segment (start 155.76 113.6) (end 147.4 113.6) (width 0.2) (layer "B.Cu") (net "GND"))
 (segment (start 164.8183 113.6) (end 155.76 113.6) (width 0.2) (layer "B.Cu") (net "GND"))
 (segment (start 147.4 113.6) (end 144 117) (width 0.2) (layer "B.Cu") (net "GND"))
 (segment (start 103.0948 117.0948) (end 103 117) (width 0.2) (layer "B.Cu") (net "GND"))
 (segment (start 144 100.42) (end 144 117) (width 0.2) (layer "B.Cu") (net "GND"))
 (segment (start 103.0948 137.2152) (end 103.0948 117.0948) (width 0.2) (layer "B.Cu") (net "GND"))
 (segment (start 142 98.42) (end 144 100.42) (width 0.2) (layer "B.Cu") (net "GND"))
 (segment (start 123.35 116.96) (end 123.4246 117.0346) (width 0.2) (layer "B.Cu") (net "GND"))
 (segment (start 169.8983 108.52) (end 164.8183 113.6) (width 0.2) (layer "B.Cu") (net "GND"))
 (segment (start 145.5034 115.1243) (end 101.0657 115.1243) (width 0.2) (layer "F.Cu") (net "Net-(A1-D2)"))
 (segment (start 146.5191 116.14) (end 145.5034 115.1243) (width 0.2) (layer "F.Cu") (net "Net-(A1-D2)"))
 (segment (start 155.76 116.14) (end 154.6583 116.14) (width 0.2) (layer "F.Cu") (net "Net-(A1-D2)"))
 (segment (start 101.0657 115.1243) (end 96.65 119.54) (width 0.2) (layer "F.Cu") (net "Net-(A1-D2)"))
 (segment (start 154.6583 116.14) (end 146.5191 116.14) (width 0.2) (layer "F.Cu") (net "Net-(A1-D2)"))
 (segment (start 151.0983 125.0334) (end 111.4666 125.0334) (width 0.2) (layer "F.Cu") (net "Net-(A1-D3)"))
 (segment (start 152.9964 123.1353) (end 151.0983 125.0334) (width 0.2) (layer "F.Cu") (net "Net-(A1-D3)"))
 (segment (start 111.4666 125.0334) (end 96.5 140) (width 0.2) (layer "F.Cu") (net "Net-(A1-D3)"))
 (via (at 152.9964 123.1353) (size 0.6) (drill 0.3) (layers "F.Cu" "B.Cu") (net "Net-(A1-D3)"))
 (segment (start 152.9964 122.4076) (end 152.9964 123.1353) (width 0.2) (layer "B.Cu") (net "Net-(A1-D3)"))
 (segment (start 155.76 119.7817) (end 155.6223 119.7817) (width 0.2) (layer "B.Cu") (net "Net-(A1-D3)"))
 (segment (start 155.6223 119.7817) (end 152.9964 122.4076) (width 0.2) (layer "B.Cu") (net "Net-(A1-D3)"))
 (segment (start 155.76 118.68) (end 155.76 119.7817) (width 0.2) (layer "B.Cu") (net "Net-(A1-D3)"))
 (segment (start 154.6583 121.22) (end 152.4869 119.0486) (width 0.2) (layer "F.Cu") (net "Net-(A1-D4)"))
 (segment (start 155.76 121.22) (end 154.6583 121.22) (width 0.2) (layer "F.Cu") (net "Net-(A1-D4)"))
 (segment (start 126.178 118.3917) (end 118.1083 118.3917) (width 0.2) (layer "F.Cu") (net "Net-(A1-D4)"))
 (segment (start 152.4869 119.0486) (end 140.8699 119.0486) (width 0.2) (layer "F.Cu") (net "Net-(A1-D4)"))
 (segment (start 139.9241 118.1028) (end 126.4669 118.1028) (width 0.2) (layer "F.Cu") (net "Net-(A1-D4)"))
 (segment (start 118.1083 118.3917) (end 117 119.5) (width 0.2) (layer "F.Cu") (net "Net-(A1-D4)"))
 (segment (start 140.8699 119.0486) (end 139.9241 118.1028) (width 0.2) (layer "F.Cu") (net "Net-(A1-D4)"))
 (segment (start 126.4669 118.1028) (end 126.178 118.3917) (width 0.2) (layer "F.Cu") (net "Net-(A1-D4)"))
 (segment (start 152.9832 125.4351) (end 154.6583 123.76) (width 0.2) (layer "F.Cu") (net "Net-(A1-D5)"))
 (segment (start 131.5649 125.4351) (end 152.9832 125.4351) (width 0.2) (layer "F.Cu") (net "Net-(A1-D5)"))
 (segment (start 155.76 123.76) (end 154.6583 123.76) (width 0.2) (layer "F.Cu") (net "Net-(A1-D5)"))
 (segment (start 117 140) (end 131.5649 125.4351) (width 0.2) (layer "F.Cu") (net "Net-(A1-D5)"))
 (segment (start 137.8325 119.7225) (end 137.65 119.54) (width 0.2) (layer "F.Cu") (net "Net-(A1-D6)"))
 (segment (start 137.8325 122.0611) (end 137.8325 119.7225) (width 0.2) (layer "F.Cu") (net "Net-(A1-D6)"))
 (segment (start 149.4527 122.5336) (end 147.5881 120.669) (width 0.2) (layer "F.Cu") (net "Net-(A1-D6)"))
 (segment (start 144.0117 123.137) (end 142.517 124.6317) (width 0.2) (layer "F.Cu") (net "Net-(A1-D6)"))
 (segment (start 140.4031 124.6317) (end 137.8325 122.0611) (width 0.2) (layer "F.Cu") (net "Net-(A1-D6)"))
 (segment (start 144.0117 122.6084) (end 144.0117 123.137) (width 0.2) (layer "F.Cu") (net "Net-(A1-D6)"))
 (segment (start 156.1219 122.5336) (end 149.4527 122.5336) (width 0.2) (layer "F.Cu") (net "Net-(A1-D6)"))
 (segment (start 155.76 125.1983) (end 155.8977 125.1983) (width 0.2) (layer "F.Cu") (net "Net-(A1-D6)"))
 (segment (start 155.8977 125.1983) (end 156.8932 124.2028) (width 0.2) (layer "F.Cu") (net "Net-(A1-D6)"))
 (segment (start 145.9511 120.669) (end 144.0117 122.6084) (width 0.2) (layer "F.Cu") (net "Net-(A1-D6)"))
 (segment (start 142.517 124.6317) (end 140.4031 124.6317) (width 0.2) (layer "F.Cu") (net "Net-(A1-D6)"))
 (segment (start 156.8932 123.3049) (end 156.1219 122.5336) (width 0.2) (layer "F.Cu") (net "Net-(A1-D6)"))
 (segment (start 155.76 126.3) (end 155.76 125.1983) (width 0.2) (layer "F.Cu") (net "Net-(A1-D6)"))
 (segment (start 156.8932 124.2028) (end 156.8932 123.3049) (width 0.2) (layer "F.Cu") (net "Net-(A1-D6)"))
 (segment (start 147.5881 120.669) (end 145.9511 120.669) (width 0.2) (layer "F.Cu") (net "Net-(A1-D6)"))
 (segment (start 155.76 128.84) (end 148.85 128.84) (width 0.2) (layer "B.Cu") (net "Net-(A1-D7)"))
 (segment (start 148.85 128.84) (end 137.65 140.04) (width 0.2) (layer "B.Cu") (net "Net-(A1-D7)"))
 (segment (start 149.5305 120.5202) (end 154.0403 125.03) (width 0.2) (layer "B.Cu") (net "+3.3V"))
 (segment (start 145.4987 120.5202) (end 149.5305 120.5202) (width 0.2) (layer "B.Cu") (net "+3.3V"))
 (segment (start 142 100.96) (end 143.1517 102.1117) (width 0.2) (layer "B.Cu") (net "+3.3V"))
 (segment (start 169.8983 138.7717) (end 169.8983 139) (width 0.2) (layer "B.Cu") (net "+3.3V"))
 (segment (start 143.1517 102.1117) (end 143.1517 114.1961) (width 0.2) (layer "B.Cu") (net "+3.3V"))
 (segment (start 154.0403 125.03) (end 156.1566 125.03) (width 0.2) (layer "B.Cu") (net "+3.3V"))
 (segment (start 171 139) (end 169.8983 139) (width 0.2) (layer "B.Cu") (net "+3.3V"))
 (segment (start 156.1566 125.03) (end 169.8983 138.7717) (width 0.2) (layer "B.Cu") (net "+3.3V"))
 (segment (start 142.5835 114.7643) (end 142.5835 117.605) (width 0.2) (layer "B.Cu") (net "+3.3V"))
 (segment (start 143.1517 114.1961) (end 142.5835 114.7643) (width 0.2) (layer "B.Cu") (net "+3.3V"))
 (segment (start 142.5835 117.605) (end 145.4987 120.5202) (width 0.2) (layer "B.Cu") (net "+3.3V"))
 (segment (start 161.0083 114.87) (end 150.83 114.87) (width 0.2) (layer "F.Cu") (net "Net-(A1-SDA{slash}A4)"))
 (segment (start 171 123.76) (end 169.8983 123.76) (width 0.2) (layer "F.Cu") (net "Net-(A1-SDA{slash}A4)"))
 (segment (start 169.8983 123.76) (end 161.0083 114.87) (width 0.2) (layer "F.Cu") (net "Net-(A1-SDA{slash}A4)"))
 (segment (start 150.83 114.87) (end 142 106.04) (width 0.2) (layer "F.Cu") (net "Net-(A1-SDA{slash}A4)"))
 (segment (start 150.8285 112.3285) (end 142 103.5) (width 0.2) (layer "F.Cu") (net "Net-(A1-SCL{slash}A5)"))
 (segment (start 171 121.22) (end 169.8983 121.22) (width 0.2) (layer "F.Cu") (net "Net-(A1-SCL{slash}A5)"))
 (segment (start 169.8983 121.22) (end 161.0068 112.3285) (width 0.2) (layer "F.Cu") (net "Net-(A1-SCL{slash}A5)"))
 (segment (start 161.0068 112.3285) (end 150.8285 112.3285) (width 0.2) (layer "F.Cu") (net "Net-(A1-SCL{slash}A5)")))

